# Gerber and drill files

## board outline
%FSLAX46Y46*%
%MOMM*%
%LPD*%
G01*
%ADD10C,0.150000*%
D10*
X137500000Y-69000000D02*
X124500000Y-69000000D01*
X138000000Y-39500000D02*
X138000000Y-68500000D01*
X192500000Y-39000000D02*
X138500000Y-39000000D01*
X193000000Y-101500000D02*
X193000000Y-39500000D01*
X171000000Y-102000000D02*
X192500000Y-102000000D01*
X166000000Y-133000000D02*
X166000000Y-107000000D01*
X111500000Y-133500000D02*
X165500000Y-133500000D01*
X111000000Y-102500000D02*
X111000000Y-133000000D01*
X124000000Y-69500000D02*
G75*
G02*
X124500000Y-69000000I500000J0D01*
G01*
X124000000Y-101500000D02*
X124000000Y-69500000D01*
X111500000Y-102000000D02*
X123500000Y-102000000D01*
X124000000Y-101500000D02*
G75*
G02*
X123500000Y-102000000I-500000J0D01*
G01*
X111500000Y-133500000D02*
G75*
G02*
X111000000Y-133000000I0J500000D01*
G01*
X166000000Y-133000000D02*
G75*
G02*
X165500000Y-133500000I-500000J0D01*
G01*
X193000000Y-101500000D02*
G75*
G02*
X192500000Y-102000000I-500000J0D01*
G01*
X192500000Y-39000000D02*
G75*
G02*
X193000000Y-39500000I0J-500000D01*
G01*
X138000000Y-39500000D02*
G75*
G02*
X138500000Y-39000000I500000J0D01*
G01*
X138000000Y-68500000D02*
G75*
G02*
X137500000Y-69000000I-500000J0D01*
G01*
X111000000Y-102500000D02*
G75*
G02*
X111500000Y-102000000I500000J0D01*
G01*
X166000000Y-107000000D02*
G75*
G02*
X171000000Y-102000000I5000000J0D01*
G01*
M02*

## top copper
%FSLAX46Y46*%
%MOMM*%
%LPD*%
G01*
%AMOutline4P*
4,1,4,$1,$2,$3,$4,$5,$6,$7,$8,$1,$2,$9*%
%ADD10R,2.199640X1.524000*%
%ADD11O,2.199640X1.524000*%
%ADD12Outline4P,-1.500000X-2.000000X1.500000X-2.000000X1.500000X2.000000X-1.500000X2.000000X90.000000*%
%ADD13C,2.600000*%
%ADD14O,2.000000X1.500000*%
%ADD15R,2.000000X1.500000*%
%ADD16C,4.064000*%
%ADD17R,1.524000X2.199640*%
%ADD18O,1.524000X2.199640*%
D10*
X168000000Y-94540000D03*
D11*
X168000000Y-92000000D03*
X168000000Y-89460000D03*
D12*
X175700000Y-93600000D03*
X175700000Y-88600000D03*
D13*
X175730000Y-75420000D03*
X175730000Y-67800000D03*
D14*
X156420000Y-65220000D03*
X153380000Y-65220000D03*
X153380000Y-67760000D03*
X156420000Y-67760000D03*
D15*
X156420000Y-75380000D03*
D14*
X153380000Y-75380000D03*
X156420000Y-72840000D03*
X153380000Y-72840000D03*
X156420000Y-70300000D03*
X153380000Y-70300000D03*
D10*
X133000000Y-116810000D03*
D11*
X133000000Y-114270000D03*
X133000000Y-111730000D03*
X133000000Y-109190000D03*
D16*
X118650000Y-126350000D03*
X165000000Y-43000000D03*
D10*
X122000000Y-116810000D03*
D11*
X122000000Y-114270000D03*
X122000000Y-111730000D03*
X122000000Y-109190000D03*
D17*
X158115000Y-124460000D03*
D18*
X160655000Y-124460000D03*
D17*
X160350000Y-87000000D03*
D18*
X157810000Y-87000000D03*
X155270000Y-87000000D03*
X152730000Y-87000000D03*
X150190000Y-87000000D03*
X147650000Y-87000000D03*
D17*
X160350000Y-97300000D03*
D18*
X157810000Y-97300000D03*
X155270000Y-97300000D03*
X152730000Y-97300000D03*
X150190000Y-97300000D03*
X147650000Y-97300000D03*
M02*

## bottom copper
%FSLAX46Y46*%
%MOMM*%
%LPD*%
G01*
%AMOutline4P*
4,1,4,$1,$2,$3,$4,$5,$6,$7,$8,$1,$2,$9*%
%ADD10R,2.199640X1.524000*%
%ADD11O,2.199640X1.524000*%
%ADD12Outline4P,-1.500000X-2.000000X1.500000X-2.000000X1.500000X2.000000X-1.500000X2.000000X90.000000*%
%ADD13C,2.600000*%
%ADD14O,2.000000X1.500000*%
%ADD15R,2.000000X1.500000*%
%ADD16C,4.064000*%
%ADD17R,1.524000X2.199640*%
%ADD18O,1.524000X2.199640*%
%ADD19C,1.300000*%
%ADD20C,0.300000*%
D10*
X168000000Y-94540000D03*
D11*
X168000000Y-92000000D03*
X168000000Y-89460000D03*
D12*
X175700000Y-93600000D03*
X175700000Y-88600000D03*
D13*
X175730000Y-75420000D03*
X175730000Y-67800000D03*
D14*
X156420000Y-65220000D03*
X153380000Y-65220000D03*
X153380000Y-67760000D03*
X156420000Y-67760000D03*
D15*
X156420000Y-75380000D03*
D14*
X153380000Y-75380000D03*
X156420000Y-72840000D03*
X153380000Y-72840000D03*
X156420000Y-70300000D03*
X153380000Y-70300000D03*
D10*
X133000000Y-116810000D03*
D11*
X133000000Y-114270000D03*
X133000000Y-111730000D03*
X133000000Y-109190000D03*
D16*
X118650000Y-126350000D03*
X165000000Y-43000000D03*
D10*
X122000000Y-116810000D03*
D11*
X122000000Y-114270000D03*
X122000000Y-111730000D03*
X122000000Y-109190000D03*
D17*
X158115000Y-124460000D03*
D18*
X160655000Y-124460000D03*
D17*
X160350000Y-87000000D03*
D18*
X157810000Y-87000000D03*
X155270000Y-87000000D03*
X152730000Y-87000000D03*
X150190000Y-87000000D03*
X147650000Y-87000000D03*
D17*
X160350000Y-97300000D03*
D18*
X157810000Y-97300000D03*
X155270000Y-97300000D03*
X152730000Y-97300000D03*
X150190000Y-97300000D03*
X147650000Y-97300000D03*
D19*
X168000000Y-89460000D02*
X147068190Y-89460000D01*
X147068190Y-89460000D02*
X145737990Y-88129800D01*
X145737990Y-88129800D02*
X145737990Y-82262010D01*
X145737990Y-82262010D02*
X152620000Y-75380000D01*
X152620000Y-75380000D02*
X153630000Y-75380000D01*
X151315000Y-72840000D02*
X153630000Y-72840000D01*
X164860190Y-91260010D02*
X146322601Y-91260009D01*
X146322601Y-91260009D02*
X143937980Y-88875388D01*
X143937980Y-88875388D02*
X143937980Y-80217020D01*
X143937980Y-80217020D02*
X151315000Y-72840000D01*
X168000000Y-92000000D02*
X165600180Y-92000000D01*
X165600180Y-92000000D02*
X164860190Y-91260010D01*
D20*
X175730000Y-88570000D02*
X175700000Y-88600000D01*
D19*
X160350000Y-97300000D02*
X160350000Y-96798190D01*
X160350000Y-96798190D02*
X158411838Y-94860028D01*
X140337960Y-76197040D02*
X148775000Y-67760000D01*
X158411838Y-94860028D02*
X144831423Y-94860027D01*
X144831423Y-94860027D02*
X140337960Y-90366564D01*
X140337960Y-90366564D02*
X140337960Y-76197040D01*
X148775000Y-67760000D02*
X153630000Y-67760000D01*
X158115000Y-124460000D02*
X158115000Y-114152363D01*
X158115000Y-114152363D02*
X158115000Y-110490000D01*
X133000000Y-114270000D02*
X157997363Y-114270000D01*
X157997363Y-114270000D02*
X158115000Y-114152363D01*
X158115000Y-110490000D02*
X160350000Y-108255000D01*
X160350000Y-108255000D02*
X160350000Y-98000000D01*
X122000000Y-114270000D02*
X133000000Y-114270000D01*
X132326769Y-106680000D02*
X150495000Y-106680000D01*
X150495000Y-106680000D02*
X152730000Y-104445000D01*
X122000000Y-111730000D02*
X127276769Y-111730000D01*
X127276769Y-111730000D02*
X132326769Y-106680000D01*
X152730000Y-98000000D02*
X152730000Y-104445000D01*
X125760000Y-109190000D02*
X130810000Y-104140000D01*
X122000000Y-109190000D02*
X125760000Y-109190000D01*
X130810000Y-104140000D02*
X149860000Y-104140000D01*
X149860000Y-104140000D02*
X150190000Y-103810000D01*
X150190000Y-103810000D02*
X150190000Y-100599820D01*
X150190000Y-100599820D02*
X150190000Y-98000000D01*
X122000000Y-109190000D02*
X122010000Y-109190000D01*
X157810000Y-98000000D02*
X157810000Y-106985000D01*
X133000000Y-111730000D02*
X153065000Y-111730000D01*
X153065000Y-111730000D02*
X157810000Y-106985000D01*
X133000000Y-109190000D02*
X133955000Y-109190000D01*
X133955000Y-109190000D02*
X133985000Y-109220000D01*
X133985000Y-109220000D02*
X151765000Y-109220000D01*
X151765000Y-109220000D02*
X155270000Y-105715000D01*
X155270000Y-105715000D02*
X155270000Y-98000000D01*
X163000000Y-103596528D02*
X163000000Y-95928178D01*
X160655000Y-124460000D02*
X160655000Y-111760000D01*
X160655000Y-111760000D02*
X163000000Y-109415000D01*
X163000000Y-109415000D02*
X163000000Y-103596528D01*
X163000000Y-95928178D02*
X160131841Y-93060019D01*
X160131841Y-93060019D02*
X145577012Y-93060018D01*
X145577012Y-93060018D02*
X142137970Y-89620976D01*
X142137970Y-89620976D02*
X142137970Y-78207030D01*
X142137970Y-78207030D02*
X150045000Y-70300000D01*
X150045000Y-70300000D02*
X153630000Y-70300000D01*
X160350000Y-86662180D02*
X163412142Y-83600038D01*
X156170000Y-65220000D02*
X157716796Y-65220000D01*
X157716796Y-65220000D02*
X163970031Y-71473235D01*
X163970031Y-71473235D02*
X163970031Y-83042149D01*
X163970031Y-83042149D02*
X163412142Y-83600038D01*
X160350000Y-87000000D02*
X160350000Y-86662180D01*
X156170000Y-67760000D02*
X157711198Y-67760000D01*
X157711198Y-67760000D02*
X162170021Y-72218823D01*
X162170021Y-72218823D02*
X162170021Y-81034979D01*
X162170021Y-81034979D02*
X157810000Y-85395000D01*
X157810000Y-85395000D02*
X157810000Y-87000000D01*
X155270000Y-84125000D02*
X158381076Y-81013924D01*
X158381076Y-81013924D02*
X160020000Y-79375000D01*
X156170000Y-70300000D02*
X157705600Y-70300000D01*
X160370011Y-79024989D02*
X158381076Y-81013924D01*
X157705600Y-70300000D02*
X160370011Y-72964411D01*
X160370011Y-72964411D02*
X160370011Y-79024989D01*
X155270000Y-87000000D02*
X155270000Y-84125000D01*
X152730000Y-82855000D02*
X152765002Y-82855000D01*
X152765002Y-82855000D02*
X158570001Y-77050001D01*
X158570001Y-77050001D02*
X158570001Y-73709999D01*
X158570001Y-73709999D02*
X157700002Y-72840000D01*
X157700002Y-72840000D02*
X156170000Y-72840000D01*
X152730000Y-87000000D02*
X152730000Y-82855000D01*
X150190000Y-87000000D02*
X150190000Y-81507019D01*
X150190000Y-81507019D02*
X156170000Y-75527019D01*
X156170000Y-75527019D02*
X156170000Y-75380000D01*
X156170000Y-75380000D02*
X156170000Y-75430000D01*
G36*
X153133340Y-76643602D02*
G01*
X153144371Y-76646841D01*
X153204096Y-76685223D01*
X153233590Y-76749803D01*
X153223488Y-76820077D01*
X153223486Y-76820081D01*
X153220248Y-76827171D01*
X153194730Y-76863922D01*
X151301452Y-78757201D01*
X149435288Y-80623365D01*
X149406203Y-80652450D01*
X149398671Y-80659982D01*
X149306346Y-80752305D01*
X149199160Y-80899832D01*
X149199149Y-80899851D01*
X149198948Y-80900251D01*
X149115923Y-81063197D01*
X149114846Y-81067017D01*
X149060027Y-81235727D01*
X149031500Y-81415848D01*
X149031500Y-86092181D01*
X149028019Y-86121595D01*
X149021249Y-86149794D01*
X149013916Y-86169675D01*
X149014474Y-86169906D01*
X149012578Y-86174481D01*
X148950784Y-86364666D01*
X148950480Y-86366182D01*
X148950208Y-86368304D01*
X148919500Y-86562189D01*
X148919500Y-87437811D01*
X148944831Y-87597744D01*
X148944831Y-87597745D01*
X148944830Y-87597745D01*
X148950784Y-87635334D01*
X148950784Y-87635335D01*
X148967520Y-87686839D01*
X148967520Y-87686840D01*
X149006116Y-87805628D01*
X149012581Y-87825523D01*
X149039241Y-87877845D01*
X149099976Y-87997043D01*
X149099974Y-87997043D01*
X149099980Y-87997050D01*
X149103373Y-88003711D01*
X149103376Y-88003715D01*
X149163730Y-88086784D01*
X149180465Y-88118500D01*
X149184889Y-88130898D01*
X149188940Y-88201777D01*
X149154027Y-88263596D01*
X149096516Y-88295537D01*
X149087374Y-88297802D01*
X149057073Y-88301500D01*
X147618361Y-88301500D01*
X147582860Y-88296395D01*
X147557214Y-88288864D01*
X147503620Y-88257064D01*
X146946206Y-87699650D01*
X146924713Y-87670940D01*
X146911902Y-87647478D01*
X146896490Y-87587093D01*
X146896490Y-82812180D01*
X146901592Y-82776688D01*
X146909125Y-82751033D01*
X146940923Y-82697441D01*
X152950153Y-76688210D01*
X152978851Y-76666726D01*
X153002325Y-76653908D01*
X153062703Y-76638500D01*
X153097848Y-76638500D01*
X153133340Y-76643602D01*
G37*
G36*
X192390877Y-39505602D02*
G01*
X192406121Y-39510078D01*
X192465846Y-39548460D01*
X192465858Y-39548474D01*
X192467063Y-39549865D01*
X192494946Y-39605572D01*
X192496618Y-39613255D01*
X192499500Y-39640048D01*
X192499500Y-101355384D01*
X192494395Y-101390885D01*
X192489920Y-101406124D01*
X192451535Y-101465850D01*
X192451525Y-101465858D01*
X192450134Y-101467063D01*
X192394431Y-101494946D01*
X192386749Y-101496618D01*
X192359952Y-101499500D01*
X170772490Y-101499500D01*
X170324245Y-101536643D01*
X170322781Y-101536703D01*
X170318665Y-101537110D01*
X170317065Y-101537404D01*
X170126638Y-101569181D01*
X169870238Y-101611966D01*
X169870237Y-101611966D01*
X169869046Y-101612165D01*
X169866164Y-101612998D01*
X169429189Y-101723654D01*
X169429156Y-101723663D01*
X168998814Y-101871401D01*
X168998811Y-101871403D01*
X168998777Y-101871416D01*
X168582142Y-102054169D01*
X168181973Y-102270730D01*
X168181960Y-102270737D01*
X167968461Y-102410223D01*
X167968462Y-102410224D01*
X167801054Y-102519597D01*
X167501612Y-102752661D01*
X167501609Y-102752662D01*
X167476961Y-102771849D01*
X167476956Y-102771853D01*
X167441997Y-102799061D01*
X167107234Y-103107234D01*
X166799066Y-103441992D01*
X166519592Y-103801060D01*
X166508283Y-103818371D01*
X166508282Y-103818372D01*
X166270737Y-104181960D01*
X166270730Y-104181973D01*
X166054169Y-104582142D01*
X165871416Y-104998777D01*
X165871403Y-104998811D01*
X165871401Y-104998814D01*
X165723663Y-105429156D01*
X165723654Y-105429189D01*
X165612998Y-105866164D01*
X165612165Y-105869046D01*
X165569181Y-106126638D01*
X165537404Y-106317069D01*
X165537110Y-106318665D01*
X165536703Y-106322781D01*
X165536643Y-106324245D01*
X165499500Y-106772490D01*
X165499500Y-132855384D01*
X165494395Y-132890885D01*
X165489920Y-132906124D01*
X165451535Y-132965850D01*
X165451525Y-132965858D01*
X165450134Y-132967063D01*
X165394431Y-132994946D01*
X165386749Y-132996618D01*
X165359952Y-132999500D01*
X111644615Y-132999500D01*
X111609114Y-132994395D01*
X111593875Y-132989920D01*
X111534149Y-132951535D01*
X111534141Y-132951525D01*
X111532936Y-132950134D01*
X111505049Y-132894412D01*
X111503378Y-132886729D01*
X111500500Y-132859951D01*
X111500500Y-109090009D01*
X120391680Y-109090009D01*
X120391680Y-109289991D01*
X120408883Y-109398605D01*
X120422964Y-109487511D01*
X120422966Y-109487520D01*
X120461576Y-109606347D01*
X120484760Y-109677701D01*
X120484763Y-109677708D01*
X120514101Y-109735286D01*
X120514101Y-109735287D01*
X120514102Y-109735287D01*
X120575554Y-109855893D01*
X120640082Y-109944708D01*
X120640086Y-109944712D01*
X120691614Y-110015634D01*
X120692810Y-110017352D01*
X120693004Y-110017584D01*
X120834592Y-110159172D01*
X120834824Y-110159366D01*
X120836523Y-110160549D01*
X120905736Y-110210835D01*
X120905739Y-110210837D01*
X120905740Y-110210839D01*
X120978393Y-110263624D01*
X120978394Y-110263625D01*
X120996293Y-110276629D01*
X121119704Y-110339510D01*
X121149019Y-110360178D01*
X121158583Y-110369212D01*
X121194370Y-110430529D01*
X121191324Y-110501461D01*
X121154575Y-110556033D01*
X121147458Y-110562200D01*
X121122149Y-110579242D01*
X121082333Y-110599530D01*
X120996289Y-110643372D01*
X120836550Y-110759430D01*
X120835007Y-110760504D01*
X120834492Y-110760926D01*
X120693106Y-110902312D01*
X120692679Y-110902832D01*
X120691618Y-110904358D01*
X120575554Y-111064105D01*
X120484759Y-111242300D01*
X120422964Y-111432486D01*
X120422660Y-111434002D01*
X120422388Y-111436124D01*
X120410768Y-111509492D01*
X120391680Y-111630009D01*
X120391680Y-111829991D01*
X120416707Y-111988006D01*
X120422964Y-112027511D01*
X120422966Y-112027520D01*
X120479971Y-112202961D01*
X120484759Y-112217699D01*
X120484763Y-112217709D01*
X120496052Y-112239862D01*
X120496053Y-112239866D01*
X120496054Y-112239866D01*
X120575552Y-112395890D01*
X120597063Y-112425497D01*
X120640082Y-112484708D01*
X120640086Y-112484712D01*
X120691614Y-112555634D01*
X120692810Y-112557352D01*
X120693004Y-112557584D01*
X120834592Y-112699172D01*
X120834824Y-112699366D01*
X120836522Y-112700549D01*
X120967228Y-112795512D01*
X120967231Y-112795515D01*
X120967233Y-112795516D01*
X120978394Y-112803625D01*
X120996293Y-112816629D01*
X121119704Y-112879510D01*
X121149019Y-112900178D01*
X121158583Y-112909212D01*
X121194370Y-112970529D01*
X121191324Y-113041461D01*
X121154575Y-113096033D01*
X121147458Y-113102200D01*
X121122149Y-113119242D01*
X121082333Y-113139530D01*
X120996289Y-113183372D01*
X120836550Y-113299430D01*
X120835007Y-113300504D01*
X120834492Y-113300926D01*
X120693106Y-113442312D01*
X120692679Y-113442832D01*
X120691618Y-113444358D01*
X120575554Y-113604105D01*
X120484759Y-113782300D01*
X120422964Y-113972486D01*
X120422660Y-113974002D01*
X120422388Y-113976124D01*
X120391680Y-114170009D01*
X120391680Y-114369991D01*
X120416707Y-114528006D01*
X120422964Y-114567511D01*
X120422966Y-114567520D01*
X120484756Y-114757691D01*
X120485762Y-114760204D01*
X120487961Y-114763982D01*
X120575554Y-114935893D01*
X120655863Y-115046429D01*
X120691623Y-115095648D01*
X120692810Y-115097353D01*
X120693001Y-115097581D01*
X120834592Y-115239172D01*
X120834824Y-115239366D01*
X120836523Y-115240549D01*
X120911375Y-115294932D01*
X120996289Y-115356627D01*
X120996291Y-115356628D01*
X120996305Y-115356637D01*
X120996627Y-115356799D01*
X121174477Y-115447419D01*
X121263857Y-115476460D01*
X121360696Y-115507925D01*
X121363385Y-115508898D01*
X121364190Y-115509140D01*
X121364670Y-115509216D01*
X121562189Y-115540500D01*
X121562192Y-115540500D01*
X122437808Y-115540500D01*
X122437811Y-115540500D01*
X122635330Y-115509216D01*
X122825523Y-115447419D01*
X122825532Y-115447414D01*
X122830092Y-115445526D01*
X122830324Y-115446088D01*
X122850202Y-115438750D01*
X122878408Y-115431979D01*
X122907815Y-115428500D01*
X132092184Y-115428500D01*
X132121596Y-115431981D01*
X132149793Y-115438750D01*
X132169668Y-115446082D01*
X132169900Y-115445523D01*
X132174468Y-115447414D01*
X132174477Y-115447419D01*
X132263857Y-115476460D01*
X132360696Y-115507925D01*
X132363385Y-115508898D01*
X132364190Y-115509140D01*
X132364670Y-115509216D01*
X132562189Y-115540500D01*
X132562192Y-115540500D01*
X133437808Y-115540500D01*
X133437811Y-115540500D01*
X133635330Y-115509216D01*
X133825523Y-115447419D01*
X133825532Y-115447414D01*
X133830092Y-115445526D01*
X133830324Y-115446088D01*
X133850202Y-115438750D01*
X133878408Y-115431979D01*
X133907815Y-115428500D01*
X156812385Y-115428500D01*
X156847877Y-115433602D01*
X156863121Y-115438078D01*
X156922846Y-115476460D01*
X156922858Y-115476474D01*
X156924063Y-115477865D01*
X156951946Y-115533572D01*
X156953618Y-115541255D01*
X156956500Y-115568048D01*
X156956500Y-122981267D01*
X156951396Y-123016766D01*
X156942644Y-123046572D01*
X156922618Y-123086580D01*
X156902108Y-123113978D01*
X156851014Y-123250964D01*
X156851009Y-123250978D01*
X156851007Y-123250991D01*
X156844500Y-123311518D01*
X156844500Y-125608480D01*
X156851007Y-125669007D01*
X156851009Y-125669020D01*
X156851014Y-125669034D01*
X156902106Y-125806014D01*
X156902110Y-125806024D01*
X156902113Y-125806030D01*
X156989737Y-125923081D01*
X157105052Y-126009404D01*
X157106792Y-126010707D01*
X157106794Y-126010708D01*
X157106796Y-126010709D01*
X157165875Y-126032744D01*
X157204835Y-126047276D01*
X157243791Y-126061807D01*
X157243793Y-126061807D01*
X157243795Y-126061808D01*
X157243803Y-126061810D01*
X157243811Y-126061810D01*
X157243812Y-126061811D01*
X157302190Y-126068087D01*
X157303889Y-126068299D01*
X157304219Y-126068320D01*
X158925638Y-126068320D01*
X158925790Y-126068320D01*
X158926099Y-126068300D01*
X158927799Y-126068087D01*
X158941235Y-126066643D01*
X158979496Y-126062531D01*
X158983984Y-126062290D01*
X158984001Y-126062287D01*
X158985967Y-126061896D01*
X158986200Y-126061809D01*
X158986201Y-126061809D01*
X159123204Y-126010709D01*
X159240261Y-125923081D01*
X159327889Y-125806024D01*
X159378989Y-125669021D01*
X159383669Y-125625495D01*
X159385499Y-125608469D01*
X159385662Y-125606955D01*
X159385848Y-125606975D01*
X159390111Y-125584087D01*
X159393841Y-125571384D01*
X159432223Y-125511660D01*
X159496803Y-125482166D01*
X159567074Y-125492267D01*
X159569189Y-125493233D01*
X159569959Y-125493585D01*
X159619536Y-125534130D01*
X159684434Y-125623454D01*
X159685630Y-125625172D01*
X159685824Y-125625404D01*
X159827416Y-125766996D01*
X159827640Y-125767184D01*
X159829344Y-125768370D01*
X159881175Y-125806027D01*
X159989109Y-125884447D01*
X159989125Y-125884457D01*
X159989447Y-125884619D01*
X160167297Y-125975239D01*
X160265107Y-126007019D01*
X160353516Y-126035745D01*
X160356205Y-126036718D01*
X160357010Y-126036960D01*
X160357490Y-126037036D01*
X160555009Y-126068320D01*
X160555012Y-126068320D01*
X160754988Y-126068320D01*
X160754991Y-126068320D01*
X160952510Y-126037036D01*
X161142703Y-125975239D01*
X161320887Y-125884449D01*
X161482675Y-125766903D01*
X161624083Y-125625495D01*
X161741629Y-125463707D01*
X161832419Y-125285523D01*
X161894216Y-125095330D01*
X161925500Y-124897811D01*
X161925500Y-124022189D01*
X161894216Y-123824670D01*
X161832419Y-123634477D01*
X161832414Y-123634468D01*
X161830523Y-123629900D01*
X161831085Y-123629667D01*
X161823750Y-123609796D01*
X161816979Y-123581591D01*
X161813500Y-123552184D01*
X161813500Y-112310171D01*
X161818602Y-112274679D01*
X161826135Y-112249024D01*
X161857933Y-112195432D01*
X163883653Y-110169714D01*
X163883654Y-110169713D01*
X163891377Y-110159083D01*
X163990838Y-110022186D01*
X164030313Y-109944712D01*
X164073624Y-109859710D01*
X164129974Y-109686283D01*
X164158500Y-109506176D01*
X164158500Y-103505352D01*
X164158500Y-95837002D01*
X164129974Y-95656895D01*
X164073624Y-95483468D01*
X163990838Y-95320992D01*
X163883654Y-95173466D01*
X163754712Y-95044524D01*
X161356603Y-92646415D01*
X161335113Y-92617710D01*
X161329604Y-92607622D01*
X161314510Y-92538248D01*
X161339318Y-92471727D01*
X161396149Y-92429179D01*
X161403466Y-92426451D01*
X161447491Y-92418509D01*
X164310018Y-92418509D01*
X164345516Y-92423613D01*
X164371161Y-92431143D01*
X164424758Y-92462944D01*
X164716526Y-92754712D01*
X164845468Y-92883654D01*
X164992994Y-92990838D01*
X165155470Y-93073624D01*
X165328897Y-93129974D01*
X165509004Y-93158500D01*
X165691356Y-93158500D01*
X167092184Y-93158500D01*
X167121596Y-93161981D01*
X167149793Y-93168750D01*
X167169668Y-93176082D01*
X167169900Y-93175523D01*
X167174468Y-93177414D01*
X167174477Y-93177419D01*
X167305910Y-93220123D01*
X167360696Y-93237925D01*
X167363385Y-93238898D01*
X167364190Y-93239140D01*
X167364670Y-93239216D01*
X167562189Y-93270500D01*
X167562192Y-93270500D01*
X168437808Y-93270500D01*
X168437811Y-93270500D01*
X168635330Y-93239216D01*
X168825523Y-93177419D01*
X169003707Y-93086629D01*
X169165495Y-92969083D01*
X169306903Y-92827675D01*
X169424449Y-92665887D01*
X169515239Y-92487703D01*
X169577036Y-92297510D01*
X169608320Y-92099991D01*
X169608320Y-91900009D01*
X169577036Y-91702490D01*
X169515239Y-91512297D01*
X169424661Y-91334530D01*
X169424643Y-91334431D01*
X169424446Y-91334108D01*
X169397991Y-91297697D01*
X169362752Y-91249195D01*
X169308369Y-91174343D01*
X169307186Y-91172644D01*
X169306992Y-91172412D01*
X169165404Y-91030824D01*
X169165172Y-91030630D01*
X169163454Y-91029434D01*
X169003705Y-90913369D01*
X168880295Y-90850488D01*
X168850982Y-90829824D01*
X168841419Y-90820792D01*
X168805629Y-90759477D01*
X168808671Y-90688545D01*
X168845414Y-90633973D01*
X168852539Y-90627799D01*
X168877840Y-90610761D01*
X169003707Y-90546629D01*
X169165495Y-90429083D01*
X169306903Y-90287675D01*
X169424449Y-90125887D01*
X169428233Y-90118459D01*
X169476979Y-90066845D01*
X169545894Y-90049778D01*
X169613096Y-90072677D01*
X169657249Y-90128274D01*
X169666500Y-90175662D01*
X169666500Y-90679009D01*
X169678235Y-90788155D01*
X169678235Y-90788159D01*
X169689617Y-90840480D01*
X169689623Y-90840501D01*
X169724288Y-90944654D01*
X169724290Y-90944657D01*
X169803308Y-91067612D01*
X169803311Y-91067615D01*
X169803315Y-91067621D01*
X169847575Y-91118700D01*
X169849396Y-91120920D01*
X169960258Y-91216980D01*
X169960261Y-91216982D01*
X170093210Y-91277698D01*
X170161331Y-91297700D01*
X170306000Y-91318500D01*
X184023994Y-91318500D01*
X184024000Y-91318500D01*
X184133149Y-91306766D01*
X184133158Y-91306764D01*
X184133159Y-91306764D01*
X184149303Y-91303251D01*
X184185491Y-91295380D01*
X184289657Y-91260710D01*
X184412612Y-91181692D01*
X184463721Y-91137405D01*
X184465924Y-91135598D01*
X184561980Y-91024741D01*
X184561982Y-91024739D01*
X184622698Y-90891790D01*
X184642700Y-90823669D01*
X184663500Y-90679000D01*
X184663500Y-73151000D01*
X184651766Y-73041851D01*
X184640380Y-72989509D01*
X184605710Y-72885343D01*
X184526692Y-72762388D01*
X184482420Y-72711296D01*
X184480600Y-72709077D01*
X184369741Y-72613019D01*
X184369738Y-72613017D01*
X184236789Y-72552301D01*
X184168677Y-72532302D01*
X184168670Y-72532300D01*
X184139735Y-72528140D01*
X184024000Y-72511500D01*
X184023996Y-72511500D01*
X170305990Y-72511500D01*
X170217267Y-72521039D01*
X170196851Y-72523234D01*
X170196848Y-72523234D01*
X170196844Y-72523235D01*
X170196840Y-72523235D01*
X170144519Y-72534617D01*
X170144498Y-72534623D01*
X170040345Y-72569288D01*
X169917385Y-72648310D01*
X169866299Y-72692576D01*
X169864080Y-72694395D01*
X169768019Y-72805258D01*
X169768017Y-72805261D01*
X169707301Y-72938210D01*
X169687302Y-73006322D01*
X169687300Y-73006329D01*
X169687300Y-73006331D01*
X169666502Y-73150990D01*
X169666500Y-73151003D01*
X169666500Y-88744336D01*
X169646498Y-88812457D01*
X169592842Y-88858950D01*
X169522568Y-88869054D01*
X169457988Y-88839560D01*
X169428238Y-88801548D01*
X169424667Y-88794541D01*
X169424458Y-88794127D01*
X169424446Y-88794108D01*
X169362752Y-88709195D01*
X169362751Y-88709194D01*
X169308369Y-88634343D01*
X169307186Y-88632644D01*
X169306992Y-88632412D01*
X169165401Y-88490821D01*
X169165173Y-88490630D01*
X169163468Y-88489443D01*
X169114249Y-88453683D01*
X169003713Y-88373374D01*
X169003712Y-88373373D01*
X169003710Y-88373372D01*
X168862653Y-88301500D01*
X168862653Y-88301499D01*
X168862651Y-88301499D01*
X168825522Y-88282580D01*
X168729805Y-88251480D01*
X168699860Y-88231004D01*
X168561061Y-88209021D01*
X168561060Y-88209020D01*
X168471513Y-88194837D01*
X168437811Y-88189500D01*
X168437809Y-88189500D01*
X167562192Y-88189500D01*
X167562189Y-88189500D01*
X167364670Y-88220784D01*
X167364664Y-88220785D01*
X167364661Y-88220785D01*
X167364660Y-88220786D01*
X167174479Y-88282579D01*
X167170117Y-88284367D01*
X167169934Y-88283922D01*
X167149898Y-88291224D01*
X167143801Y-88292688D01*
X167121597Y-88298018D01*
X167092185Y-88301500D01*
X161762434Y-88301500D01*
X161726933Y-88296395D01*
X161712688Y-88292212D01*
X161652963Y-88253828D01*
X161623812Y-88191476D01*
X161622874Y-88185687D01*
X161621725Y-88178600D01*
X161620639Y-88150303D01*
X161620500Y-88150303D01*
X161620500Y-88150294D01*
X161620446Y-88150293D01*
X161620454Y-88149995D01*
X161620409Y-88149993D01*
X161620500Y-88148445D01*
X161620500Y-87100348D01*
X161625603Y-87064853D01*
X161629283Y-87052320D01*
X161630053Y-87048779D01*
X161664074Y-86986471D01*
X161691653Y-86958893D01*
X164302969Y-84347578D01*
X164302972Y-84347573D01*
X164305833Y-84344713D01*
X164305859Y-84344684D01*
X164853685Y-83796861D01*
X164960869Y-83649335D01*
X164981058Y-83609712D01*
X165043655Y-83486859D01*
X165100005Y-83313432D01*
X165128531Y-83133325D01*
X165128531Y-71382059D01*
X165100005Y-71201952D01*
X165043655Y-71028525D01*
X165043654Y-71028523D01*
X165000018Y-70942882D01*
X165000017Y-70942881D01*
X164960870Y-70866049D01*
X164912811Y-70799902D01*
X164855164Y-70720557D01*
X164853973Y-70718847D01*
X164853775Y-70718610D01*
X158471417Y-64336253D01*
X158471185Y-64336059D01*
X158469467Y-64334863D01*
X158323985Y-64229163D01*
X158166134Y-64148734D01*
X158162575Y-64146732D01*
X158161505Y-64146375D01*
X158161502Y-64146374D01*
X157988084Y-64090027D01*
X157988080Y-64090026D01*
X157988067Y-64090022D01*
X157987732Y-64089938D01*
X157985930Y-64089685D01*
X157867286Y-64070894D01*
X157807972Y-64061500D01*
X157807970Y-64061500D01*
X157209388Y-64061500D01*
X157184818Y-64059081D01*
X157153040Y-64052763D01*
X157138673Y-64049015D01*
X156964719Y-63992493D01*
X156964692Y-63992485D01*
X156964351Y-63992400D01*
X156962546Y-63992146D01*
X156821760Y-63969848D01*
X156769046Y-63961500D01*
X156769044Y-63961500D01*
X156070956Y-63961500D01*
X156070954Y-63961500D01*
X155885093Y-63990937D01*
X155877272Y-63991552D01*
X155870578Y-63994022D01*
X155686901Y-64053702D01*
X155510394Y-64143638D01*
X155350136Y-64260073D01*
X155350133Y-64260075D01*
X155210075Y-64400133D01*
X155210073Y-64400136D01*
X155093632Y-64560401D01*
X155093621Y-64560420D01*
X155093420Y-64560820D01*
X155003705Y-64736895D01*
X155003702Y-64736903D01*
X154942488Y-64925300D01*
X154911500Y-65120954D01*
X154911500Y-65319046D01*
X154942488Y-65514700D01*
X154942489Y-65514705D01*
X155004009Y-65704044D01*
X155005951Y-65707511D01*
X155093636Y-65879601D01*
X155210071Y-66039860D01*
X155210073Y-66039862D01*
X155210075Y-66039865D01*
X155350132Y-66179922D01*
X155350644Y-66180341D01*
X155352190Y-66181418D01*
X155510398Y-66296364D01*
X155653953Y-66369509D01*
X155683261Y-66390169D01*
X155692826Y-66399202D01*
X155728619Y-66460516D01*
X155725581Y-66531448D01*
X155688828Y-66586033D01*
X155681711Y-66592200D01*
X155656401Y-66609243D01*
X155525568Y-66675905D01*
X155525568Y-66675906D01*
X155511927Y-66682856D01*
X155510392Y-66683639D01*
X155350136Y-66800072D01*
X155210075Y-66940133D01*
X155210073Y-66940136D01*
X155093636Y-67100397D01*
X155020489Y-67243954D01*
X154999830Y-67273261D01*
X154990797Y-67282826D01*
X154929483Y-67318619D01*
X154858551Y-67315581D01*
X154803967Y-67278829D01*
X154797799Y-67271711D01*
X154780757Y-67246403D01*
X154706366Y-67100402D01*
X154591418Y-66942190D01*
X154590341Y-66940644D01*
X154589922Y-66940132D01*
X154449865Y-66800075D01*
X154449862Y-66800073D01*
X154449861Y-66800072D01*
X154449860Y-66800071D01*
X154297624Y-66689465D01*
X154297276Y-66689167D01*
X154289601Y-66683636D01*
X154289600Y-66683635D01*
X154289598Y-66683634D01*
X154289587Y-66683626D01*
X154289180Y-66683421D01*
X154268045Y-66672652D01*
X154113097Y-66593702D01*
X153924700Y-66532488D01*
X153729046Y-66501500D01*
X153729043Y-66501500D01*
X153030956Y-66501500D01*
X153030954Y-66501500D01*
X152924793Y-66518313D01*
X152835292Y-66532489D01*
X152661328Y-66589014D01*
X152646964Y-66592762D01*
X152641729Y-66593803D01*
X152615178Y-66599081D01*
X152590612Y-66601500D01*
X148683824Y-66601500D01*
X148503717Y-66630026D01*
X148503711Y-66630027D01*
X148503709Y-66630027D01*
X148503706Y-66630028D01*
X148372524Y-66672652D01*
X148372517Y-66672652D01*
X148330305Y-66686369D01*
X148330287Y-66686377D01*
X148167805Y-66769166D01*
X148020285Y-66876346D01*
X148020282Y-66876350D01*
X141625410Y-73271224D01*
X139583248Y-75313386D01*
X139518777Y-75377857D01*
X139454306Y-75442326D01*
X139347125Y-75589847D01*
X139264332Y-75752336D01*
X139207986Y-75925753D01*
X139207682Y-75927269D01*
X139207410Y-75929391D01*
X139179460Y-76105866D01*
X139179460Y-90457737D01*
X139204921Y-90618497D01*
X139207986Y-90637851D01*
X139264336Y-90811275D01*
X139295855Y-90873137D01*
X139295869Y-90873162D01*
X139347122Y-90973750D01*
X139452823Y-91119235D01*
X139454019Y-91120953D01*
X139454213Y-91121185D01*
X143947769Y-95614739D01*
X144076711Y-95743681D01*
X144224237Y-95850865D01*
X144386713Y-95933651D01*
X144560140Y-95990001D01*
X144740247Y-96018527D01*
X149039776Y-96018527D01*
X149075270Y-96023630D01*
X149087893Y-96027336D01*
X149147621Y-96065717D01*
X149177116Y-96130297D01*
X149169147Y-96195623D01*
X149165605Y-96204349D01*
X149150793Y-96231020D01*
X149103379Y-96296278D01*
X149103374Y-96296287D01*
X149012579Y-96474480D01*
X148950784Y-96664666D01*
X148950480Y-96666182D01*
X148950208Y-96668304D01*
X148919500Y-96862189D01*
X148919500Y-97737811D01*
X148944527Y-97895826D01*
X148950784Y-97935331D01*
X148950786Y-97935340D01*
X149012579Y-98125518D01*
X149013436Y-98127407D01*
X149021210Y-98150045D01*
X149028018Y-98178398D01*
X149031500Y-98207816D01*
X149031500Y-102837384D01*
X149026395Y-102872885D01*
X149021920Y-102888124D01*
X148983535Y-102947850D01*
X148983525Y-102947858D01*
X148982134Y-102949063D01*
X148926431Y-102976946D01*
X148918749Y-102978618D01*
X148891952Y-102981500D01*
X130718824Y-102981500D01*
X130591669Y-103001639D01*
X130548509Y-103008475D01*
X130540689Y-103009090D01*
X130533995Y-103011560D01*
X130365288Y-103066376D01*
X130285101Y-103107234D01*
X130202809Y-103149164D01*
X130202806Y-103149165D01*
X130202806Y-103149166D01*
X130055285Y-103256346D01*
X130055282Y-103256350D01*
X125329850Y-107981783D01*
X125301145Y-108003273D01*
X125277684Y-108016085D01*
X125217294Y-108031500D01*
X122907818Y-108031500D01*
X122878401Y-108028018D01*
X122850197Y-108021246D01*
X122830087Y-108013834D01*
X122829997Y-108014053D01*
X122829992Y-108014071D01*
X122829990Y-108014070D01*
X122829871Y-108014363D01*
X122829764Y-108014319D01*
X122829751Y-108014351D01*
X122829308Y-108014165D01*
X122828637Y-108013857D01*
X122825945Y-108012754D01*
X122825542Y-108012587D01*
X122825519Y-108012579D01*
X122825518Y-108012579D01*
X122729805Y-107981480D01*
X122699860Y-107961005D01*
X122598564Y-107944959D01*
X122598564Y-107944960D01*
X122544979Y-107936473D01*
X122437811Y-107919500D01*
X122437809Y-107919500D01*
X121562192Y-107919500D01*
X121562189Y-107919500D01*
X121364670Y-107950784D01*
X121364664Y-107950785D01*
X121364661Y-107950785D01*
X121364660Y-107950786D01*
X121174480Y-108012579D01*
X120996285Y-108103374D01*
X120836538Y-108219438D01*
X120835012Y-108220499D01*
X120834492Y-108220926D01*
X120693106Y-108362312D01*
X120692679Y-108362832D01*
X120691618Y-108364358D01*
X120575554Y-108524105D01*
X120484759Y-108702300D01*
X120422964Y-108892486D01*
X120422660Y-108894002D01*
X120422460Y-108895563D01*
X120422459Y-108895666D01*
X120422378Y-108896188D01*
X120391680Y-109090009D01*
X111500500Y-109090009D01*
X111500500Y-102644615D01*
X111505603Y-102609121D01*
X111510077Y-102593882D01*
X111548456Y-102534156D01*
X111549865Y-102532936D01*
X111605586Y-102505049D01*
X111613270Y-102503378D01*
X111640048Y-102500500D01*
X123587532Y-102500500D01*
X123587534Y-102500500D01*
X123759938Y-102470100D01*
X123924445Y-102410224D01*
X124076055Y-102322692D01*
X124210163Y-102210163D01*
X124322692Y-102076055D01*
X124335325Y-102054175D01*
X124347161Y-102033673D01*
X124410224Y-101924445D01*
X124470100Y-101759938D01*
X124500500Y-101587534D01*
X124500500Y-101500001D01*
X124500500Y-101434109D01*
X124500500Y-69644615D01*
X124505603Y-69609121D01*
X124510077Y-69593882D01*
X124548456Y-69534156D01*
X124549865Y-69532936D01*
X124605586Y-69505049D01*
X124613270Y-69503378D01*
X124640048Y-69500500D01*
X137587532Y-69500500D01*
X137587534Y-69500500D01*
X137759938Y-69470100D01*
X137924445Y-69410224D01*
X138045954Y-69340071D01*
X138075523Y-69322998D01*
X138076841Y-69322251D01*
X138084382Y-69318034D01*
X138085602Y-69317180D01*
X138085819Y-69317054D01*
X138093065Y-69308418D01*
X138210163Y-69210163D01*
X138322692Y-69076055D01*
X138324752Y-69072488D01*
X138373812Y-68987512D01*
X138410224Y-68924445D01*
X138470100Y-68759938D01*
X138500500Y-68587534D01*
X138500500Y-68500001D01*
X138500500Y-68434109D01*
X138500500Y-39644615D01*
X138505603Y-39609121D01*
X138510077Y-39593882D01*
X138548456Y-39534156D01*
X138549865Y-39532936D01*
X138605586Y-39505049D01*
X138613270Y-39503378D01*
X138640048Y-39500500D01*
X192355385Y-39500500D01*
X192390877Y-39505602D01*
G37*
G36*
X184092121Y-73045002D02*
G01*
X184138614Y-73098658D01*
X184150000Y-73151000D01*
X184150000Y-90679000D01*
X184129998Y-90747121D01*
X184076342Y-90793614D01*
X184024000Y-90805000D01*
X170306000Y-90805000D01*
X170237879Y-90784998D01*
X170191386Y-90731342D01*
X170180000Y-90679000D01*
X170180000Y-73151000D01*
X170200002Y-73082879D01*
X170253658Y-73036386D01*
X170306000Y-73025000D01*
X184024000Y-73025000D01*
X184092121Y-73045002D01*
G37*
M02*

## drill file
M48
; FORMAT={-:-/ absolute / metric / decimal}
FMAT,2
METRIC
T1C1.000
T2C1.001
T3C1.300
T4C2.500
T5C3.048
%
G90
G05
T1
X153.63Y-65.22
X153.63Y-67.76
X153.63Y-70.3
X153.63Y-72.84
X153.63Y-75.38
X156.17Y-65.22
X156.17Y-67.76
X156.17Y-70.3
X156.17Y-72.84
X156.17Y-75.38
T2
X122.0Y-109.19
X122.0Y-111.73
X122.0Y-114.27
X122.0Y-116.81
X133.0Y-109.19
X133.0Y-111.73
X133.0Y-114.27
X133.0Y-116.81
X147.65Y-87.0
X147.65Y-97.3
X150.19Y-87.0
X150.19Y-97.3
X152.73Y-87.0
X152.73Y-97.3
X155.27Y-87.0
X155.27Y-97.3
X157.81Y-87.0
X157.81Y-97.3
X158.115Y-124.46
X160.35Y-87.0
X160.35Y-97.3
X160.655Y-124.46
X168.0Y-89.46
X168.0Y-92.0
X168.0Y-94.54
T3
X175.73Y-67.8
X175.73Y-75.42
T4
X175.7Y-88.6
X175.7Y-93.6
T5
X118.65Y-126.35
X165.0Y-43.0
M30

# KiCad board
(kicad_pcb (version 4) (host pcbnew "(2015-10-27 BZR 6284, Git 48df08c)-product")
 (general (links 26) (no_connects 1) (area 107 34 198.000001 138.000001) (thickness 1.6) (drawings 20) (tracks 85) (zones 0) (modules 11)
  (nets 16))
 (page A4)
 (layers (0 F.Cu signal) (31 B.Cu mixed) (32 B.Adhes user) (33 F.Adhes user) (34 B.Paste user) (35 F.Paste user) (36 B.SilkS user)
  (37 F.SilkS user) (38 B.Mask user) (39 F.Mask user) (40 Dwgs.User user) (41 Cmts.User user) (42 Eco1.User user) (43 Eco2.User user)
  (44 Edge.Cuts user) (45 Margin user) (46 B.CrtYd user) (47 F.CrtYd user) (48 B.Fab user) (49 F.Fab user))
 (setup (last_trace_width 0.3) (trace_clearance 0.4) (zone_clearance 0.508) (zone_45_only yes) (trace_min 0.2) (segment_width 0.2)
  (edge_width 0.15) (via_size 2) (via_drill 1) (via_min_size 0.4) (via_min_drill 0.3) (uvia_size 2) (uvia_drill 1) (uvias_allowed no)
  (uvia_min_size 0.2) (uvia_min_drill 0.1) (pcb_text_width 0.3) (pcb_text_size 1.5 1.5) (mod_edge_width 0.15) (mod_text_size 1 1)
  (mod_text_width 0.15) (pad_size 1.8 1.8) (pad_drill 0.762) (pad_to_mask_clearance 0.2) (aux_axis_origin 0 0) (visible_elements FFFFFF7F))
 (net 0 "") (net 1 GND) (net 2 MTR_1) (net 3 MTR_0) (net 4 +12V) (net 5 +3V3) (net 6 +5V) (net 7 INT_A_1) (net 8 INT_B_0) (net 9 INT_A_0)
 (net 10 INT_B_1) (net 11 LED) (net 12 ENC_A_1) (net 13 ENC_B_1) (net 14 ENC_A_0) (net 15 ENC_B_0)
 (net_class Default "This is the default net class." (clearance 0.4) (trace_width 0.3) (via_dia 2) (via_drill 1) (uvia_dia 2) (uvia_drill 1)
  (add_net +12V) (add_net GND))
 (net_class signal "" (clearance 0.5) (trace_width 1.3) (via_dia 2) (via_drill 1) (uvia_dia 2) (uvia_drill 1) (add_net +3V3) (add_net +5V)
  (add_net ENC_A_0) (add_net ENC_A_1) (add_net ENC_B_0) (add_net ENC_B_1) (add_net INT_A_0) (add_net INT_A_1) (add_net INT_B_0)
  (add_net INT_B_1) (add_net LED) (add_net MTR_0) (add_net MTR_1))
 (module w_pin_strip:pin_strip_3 (layer F.Cu) (at 168 92 90)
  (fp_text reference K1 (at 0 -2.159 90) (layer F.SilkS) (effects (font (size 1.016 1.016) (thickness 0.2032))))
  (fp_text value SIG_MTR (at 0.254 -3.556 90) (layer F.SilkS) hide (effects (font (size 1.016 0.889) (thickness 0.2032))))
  (pad 1 thru_hole rect (at -2.54 0 90) (size 1.524 2.19964) (drill 1.00076) (layers *.Cu *.Mask F.SilkS) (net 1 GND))
  (pad 2 thru_hole oval (at 0 0 90) (size 1.524 2.19964) (drill 1.00076) (layers *.Cu *.Mask F.SilkS) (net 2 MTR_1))
  (pad 3 thru_hole oval (at 2.54 0 90) (size 1.524 2.19964) (drill 1.00076) (layers *.Cu *.Mask F.SilkS) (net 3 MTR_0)))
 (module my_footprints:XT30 (layer F.Cu) (at 175.7 91.1 90)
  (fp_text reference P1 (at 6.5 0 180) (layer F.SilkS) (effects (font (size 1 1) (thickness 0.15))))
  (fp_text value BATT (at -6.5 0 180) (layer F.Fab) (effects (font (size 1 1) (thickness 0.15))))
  (pad 1 thru_hole trapezoid (at -2.5 0 90) (size 3 4) (drill 2.5) (layers *.Cu *.Mask F.SilkS) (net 1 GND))
  (pad 2 thru_hole trapezoid (at 2.5 0 90) (size 3 4) (drill 2.5) (layers *.Cu *.Mask F.SilkS) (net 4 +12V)))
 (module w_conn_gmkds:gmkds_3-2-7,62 (layer F.Cu) (at 175.73 71.61 90)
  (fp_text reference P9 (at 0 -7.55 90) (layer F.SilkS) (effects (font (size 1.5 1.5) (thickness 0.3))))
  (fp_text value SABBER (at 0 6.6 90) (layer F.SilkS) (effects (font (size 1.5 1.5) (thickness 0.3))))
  (pad 1 thru_hole circle (at -3.81 0 90) (size 2.6 2.6) (drill 1.3) (layers *.Cu *.Mask F.SilkS) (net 4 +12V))
  (pad 2 thru_hole circle (at 3.81 0 90) (size 2.6 2.6) (drill 1.3) (layers *.Cu *.Mask F.SilkS) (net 1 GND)))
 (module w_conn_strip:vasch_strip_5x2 (layer F.Cu) (at 154.9 70.3 90)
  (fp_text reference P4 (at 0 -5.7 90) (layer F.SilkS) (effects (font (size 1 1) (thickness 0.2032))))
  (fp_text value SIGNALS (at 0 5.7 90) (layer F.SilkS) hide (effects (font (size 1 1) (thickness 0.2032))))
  (pad 9 thru_hole oval (at 5.08 1.27 90) (size 1.5 2) (drill 1 (offset 0 0.25)) (layers *.Cu *.Mask F.SilkS) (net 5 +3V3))
  (pad 10 thru_hole oval (at 5.08 -1.27 90) (size 1.5 2) (drill 1 (offset 0 -0.25)) (layers *.Cu *.Mask F.SilkS) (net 1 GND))
  (pad 8 thru_hole oval (at 2.54 -1.27 90) (size 1.5 2) (drill 1 (offset 0 -0.25)) (layers *.Cu *.Mask F.SilkS) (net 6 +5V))
  (pad 7 thru_hole oval (at 2.54 1.27 90) (size 1.5 2) (drill 1 (offset 0 0.25)) (layers *.Cu *.Mask F.SilkS) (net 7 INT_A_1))
  (pad 1 thru_hole rect (at -5.08 1.27 90) (size 1.5 2) (drill 1 (offset 0 0.25)) (layers *.Cu *.Mask F.SilkS) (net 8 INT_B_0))
  (pad 2 thru_hole oval (at -5.08 -1.27 90) (size 1.5 2) (drill 1 (offset 0 -0.25)) (layers *.Cu *.Mask F.SilkS) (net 3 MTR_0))
  (pad 3 thru_hole oval (at -2.54 1.27 90) (size 1.5 2) (drill 1 (offset 0 0.25)) (layers *.Cu *.Mask F.SilkS) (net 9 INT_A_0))
  (pad 4 thru_hole oval (at -2.54 -1.27 90) (size 1.5 2) (drill 1 (offset 0 -0.25)) (layers *.Cu *.Mask F.SilkS) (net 2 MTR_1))
  (pad 5 thru_hole oval (at 0 1.27 90) (size 1.5 2) (drill 1 (offset 0 0.25)) (layers *.Cu *.Mask F.SilkS) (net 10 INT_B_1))
  (pad 6 thru_hole oval (at 0 -1.27 90) (size 1.5 2) (drill 1 (offset 0 -0.25)) (layers *.Cu *.Mask F.SilkS) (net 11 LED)))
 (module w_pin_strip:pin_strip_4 (layer F.Cu) (at 133 113 90)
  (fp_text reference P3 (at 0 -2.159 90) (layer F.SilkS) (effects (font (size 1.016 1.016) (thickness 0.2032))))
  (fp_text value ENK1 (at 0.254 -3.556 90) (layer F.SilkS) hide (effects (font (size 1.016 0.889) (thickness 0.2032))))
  (pad 1 thru_hole rect (at -3.81 0 90) (size 1.524 2.19964) (drill 1.00076) (layers *.Cu *.Mask F.SilkS) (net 1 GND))
  (pad 2 thru_hole oval (at -1.27 0 90) (size 1.524 2.19964) (drill 1.00076) (layers *.Cu *.Mask F.SilkS) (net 6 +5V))
  (pad 3 thru_hole oval (at 1.27 0 90) (size 1.524 2.19964) (drill 1.00076) (layers *.Cu *.Mask F.SilkS) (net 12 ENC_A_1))
  (pad 4 thru_hole oval (at 3.81 0 90) (size 1.524 2.19964) (drill 1.00076) (layers *.Cu *.Mask F.SilkS) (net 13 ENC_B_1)))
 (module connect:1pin (layer F.Cu) (at 118.65 126.35)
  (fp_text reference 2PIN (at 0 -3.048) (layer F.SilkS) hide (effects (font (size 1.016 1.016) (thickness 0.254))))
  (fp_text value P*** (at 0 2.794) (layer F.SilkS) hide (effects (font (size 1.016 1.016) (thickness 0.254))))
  (pad 1 thru_hole circle (at 0 0) (size 4.064 4.064) (drill 3.048) (layers *.Cu *.Mask F.SilkS) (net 1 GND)))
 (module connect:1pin (layer F.Cu) (at 165 43)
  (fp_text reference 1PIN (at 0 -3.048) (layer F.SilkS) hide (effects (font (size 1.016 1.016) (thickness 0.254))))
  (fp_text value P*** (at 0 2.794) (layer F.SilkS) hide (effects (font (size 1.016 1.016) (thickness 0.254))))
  (pad 2 thru_hole circle (at 0 0) (size 4.064 4.064) (drill 3.048) (layers *.Cu *.Mask F.SilkS) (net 1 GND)))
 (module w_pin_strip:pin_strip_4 (layer F.Cu) (at 122 113 90)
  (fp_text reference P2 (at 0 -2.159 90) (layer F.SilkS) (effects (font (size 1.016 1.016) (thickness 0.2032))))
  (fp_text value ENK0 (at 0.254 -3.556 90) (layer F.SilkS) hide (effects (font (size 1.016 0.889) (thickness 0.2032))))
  (pad 1 thru_hole rect (at -3.81 0 90) (size 1.524 2.19964) (drill 1.00076) (layers *.Cu *.Mask F.SilkS) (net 1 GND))
  (pad 2 thru_hole oval (at -1.27 0 90) (size 1.524 2.19964) (drill 1.00076) (layers *.Cu *.Mask F.SilkS) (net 6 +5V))
  (pad 3 thru_hole oval (at 1.27 0 90) (size 1.524 2.19964) (drill 1.00076) (layers *.Cu *.Mask F.SilkS) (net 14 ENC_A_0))
  (pad 4 thru_hole oval (at 3.81 0 90) (size 1.524 2.19964) (drill 1.00076) (layers *.Cu *.Mask F.SilkS) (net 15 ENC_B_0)))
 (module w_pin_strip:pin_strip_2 (layer F.Cu) (at 159.385 124.46)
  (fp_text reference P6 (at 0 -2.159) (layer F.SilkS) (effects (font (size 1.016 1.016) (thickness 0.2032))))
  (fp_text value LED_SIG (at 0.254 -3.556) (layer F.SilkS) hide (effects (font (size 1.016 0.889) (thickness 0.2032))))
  (pad 1 thru_hole rect (at -1.27 0) (size 1.524 2.19964) (drill 1.00076) (layers *.Cu *.Mask F.SilkS) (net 6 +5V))
  (pad 2 thru_hole oval (at 1.27 0) (size 1.524 2.19964) (drill 1.00076) (layers *.Cu *.Mask F.SilkS) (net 11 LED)))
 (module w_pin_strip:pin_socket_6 (layer F.Cu) (at 154 87 180)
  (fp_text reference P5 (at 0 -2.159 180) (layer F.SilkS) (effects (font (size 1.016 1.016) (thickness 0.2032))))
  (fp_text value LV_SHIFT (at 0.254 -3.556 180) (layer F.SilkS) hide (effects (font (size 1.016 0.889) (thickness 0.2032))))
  (pad 1 thru_hole rect (at -6.35 0 180) (size 1.524 2.19964) (drill 1.00076) (layers *.Cu *.Mask F.SilkS) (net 5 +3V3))
  (pad 2 thru_hole oval (at -3.81 0 180) (size 1.524 2.19964) (drill 1.00076) (layers *.Cu *.Mask F.SilkS) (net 7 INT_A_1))
  (pad 3 thru_hole oval (at -1.27 0 180) (size 1.524 2.19964) (drill 1.00076) (layers *.Cu *.Mask F.SilkS) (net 10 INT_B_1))
  (pad 4 thru_hole oval (at 1.27 0 180) (size 1.524 2.19964) (drill 1.00076) (layers *.Cu *.Mask F.SilkS) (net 9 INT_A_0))
  (pad 5 thru_hole oval (at 3.81 0 180) (size 1.524 2.19964) (drill 1.00076) (layers *.Cu *.Mask F.SilkS) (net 8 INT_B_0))
  (pad 6 thru_hole oval (at 6.35 0 180) (size 1.524 2.19964) (drill 1.00076) (layers *.Cu *.Mask F.SilkS) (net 1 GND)))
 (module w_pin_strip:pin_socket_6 (layer F.Cu) (at 154 97.3 180)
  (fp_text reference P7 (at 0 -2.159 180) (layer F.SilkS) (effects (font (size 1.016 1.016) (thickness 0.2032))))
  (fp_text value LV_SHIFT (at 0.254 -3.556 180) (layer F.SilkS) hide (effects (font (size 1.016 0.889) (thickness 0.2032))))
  (pad 1 thru_hole rect (at -6.35 0 180) (size 1.524 2.19964) (drill 1.00076) (layers *.Cu *.Mask F.SilkS) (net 6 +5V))
  (pad 2 thru_hole oval (at -3.81 0 180) (size 1.524 2.19964) (drill 1.00076) (layers *.Cu *.Mask F.SilkS) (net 12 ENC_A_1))
  (pad 3 thru_hole oval (at -1.27 0 180) (size 1.524 2.19964) (drill 1.00076) (layers *.Cu *.Mask F.SilkS) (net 13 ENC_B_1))
  (pad 4 thru_hole oval (at 1.27 0 180) (size 1.524 2.19964) (drill 1.00076) (layers *.Cu *.Mask F.SilkS) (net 14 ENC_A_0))
  (pad 5 thru_hole oval (at 3.81 0 180) (size 1.524 2.19964) (drill 1.00076) (layers *.Cu *.Mask F.SilkS) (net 15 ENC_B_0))
  (pad 6 thru_hole oval (at 6.35 0 180) (size 1.524 2.19964) (drill 1.00076) (layers *.Cu *.Mask F.SilkS) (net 1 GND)))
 (gr_line (start 137.5 69) (end 124.5 69) (angle 90) (layer Edge.Cuts) (width 0.15))
 (gr_line (start 138 39.5) (end 138 68.5) (angle 90) (layer Edge.Cuts) (width 0.15))
 (gr_line (start 192.5 39) (end 138.5 39) (angle 90) (layer Edge.Cuts) (width 0.15))
 (gr_line (start 193 101.5) (end 193 39.5) (angle 90) (layer Edge.Cuts) (width 0.15))
 (gr_line (start 171 102) (end 192.5 102) (angle 90) (layer Edge.Cuts) (width 0.15))
 (gr_line (start 166 133) (end 166 107) (angle 90) (layer Edge.Cuts) (width 0.15))
 (gr_line (start 111.5 133.5) (end 165.5 133.5) (angle 90) (layer Edge.Cuts) (width 0.15))
 (gr_line (start 111 102.5) (end 111 133) (angle 90) (layer Edge.Cuts) (width 0.15))
 (gr_arc (start 124.5 69.5) (end 124 69.5) (angle 90) (layer Edge.Cuts) (width 0.15))
 (gr_line (start 124 101.5) (end 124 69.5) (angle 90) (layer Edge.Cuts) (width 0.15))
 (gr_line (start 111.5 102) (end 123.5 102) (angle 90) (layer Edge.Cuts) (width 0.15))
 (gr_arc (start 123.5 101.5) (end 124 101.5) (angle 90) (layer Edge.Cuts) (width 0.15))
 (gr_arc (start 111.5 133) (end 111.5 133.5) (angle 90) (layer Edge.Cuts) (width 0.15))
 (gr_arc (start 165.5 133) (end 166 133) (angle 90) (layer Edge.Cuts) (width 0.15))
 (gr_arc (start 192.5 101.5) (end 193 101.5) (angle 90) (layer Edge.Cuts) (width 0.15))
 (gr_arc (start 192.5 39.5) (end 192.5 39) (angle 90) (layer Edge.Cuts) (width 0.15))
 (gr_arc (start 138.5 39.5) (end 138 39.5) (angle 90) (layer Edge.Cuts) (width 0.15))
 (gr_arc (start 137.5 68.5) (end 138 68.5) (angle 90) (layer Edge.Cuts) (width 0.15))
 (gr_arc (start 111.5 102.5) (end 111 102.5) (angle 90) (layer Edge.Cuts) (width 0.15))
 (gr_arc (start 171 107) (end 166 107) (angle 90) (layer Edge.Cuts) (width 0.15))
 (segment (start 168 89.46) (end 147.06819 89.46) (width 1.3) (layer B.Cu) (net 3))
 (segment (start 147.06819 89.46) (end 145.73799 88.1298) (width 1.3) (layer B.Cu) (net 3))
 (segment (start 145.73799 88.1298) (end 145.73799 82.26201) (width 1.3) (layer B.Cu) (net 3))
 (segment (start 145.73799 82.26201) (end 152.62 75.38) (width 1.3) (layer B.Cu) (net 3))
 (segment (start 152.62 75.38) (end 153.63 75.38) (width 1.3) (layer B.Cu) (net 3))
 (segment (start 151.315 72.84) (end 153.63 72.84) (width 1.3) (layer B.Cu) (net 2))
 (segment (start 164.86019 91.26001) (end 146.322601 91.260009) (width 1.3) (layer B.Cu) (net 2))
 (segment (start 146.322601 91.260009) (end 143.93798 88.875388) (width 1.3) (layer B.Cu) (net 2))
 (segment (start 143.93798 88.875388) (end 143.93798 80.21702) (width 1.3) (layer B.Cu) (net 2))
 (segment (start 143.93798 80.21702) (end 151.315 72.84) (width 1.3) (layer B.Cu) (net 2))
 (segment (start 168 92) (end 165.60018 92) (width 1.3) (layer B.Cu) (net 2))
 (segment (start 165.60018 92) (end 164.86019 91.26001) (width 1.3) (layer B.Cu) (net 2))
 (segment (start 175.73 88.57) (end 175.7 88.6) (width 0.3) (layer B.Cu) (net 4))
 (segment (start 160.35 97.3) (end 160.35 96.79819) (width 1.3) (layer B.Cu) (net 6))
 (segment (start 160.35 96.79819) (end 158.411838 94.860028) (width 1.3) (layer B.Cu) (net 6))
 (segment (start 140.33796 76.19704) (end 148.775 67.76) (width 1.3) (layer B.Cu) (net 6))
 (segment (start 158.411838 94.860028) (end 144.831423 94.860027) (width 1.3) (layer B.Cu) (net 6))
 (segment (start 144.831423 94.860027) (end 140.33796 90.366564) (width 1.3) (layer B.Cu) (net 6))
 (segment (start 140.33796 90.366564) (end 140.33796 76.19704) (width 1.3) (layer B.Cu) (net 6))
 (segment (start 148.775 67.76) (end 153.63 67.76) (width 1.3) (layer B.Cu) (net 6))
 (segment (start 158.115 124.46) (end 158.115 114.152363) (width 1.3) (layer B.Cu) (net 6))
 (segment (start 158.115 114.152363) (end 158.115 110.49) (width 1.3) (layer B.Cu) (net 6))
 (segment (start 133 114.27) (end 157.997363 114.27) (width 1.3) (layer B.Cu) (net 6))
 (segment (start 157.997363 114.27) (end 158.115 114.152363) (width 1.3) (layer B.Cu) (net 6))
 (segment (start 158.115 110.49) (end 160.35 108.255) (width 1.3) (layer B.Cu) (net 6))
 (segment (start 160.35 108.255) (end 160.35 98) (width 1.3) (layer B.Cu) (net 6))
 (segment (start 122 114.27) (end 133 114.27) (width 1.3) (layer B.Cu) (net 6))
 (segment (start 132.326769 106.68) (end 150.495 106.68) (width 1.3) (layer B.Cu) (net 14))
 (segment (start 150.495 106.68) (end 152.73 104.445) (width 1.3) (layer B.Cu) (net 14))
 (segment (start 122 111.73) (end 127.276769 111.73) (width 1.3) (layer B.Cu) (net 14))
 (segment (start 127.276769 111.73) (end 132.326769 106.68) (width 1.3) (layer B.Cu) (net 14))
 (segment (start 152.73 98) (end 152.73 104.445) (width 1.3) (layer B.Cu) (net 14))
 (segment (start 125.76 109.19) (end 130.81 104.14) (width 1.3) (layer B.Cu) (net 15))
 (segment (start 122 109.19) (end 125.76 109.19) (width 1.3) (layer B.Cu) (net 15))
 (segment (start 130.81 104.14) (end 149.86 104.14) (width 1.3) (layer B.Cu) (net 15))
 (segment (start 149.86 104.14) (end 150.19 103.81) (width 1.3) (layer B.Cu) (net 15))
 (segment (start 150.19 103.81) (end 150.19 100.59982) (width 1.3) (layer B.Cu) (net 15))
 (segment (start 150.19 100.59982) (end 150.19 98) (width 1.3) (layer B.Cu) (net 15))
 (segment (start 122 109.19) (end 122.01 109.19) (width 1.3) (layer B.Cu) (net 15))
 (segment (start 157.81 98) (end 157.81 106.985) (width 1.3) (layer B.Cu) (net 12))
 (segment (start 133 111.73) (end 153.065 111.73) (width 1.3) (layer B.Cu) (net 12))
 (segment (start 153.065 111.73) (end 157.81 106.985) (width 1.3) (layer B.Cu) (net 12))
 (segment (start 133 109.19) (end 133.955 109.19) (width 1.3) (layer B.Cu) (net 13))
 (segment (start 133.955 109.19) (end 133.985 109.22) (width 1.3) (layer B.Cu) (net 13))
 (segment (start 133.985 109.22) (end 151.765 109.22) (width 1.3) (layer B.Cu) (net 13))
 (segment (start 151.765 109.22) (end 155.27 105.715) (width 1.3) (layer B.Cu) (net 13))
 (segment (start 155.27 105.715) (end 155.27 98) (width 1.3) (layer B.Cu) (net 13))
 (segment (start 163 103.596528) (end 163 95.928178) (width 1.3) (layer B.Cu) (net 11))
 (segment (start 160.655 124.46) (end 160.655 111.76) (width 1.3) (layer B.Cu) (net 11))
 (segment (start 160.655 111.76) (end 163 109.415) (width 1.3) (layer B.Cu) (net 11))
 (segment (start 163 109.415) (end 163 103.596528) (width 1.3) (layer B.Cu) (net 11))
 (segment (start 163 95.928178) (end 160.131841 93.060019) (width 1.3) (layer B.Cu) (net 11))
 (segment (start 160.131841 93.060019) (end 145.577012 93.060018) (width 1.3) (layer B.Cu) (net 11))
 (segment (start 145.577012 93.060018) (end 142.13797 89.620976) (width 1.3) (layer B.Cu) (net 11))
 (segment (start 142.13797 89.620976) (end 142.13797 78.20703) (width 1.3) (layer B.Cu) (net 11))
 (segment (start 142.13797 78.20703) (end 150.045 70.3) (width 1.3) (layer B.Cu) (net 11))
 (segment (start 150.045 70.3) (end 153.63 70.3) (width 1.3) (layer B.Cu) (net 11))
 (segment (start 160.35 86.66218) (end 163.412142 83.600038) (width 1.3) (layer B.Cu) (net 5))
 (segment (start 156.17 65.22) (end 157.716796 65.22) (width 1.3) (layer B.Cu) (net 5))
 (segment (start 157.716796 65.22) (end 163.970031 71.473235) (width 1.3) (layer B.Cu) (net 5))
 (segment (start 163.970031 71.473235) (end 163.970031 83.042149) (width 1.3) (layer B.Cu) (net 5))
 (segment (start 163.970031 83.042149) (end 163.412142 83.600038) (width 1.3) (layer B.Cu) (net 5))
 (segment (start 160.35 87) (end 160.35 86.66218) (width 1.3) (layer B.Cu) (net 5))
 (segment (start 156.17 67.76) (end 157.711198 67.76) (width 1.3) (layer B.Cu) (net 7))
 (segment (start 157.711198 67.76) (end 162.170021 72.218823) (width 1.3) (layer B.Cu) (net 7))
 (segment (start 162.170021 72.218823) (end 162.170021 81.034979) (width 1.3) (layer B.Cu) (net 7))
 (segment (start 162.170021 81.034979) (end 157.81 85.395) (width 1.3) (layer B.Cu) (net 7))
 (segment (start 157.81 85.395) (end 157.81 87) (width 1.3) (layer B.Cu) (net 7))
 (segment (start 155.27 84.125) (end 158.381076 81.013924) (width 1.3) (layer B.Cu) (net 10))
 (segment (start 158.381076 81.013924) (end 160.02 79.375) (width 1.3) (layer B.Cu) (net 10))
 (segment (start 156.17 70.3) (end 157.7056 70.3) (width 1.3) (layer B.Cu) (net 10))
 (segment (start 160.370011 79.024989) (end 158.381076 81.013924) (width 1.3) (layer B.Cu) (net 10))
 (segment (start 157.7056 70.3) (end 160.370011 72.964411) (width 1.3) (layer B.Cu) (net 10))
 (segment (start 160.370011 72.964411) (end 160.370011 79.024989) (width 1.3) (layer B.Cu) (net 10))
 (segment (start 155.27 87) (end 155.27 84.125) (width 1.3) (layer B.Cu) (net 10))
 (segment (start 152.73 82.855) (end 152.765002 82.855) (width 1.3) (layer B.Cu) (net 9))
 (segment (start 152.765002 82.855) (end 158.570001 77.050001) (width 1.3) (layer B.Cu) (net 9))
 (segment (start 158.570001 77.050001) (end 158.570001 73.709999) (width 1.3) (layer B.Cu) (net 9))
 (segment (start 158.570001 73.709999) (end 157.700002 72.84) (width 1.3) (layer B.Cu) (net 9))
 (segment (start 157.700002 72.84) (end 156.17 72.84) (width 1.3) (layer B.Cu) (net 9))
 (segment (start 152.73 87) (end 152.73 82.855) (width 1.3) (layer B.Cu) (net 9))
 (segment (start 150.19 87) (end 150.19 81.507019) (width 1.3) (layer B.Cu) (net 8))
 (segment (start 150.19 81.507019) (end 156.17 75.527019) (width 1.3) (layer B.Cu) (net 8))
 (segment (start 156.17 75.527019) (end 156.17 75.38) (width 1.3) (layer B.Cu) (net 8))
 (segment (start 156.17 75.38) (end 156.17 75.43) (width 1.3) (layer B.Cu) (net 8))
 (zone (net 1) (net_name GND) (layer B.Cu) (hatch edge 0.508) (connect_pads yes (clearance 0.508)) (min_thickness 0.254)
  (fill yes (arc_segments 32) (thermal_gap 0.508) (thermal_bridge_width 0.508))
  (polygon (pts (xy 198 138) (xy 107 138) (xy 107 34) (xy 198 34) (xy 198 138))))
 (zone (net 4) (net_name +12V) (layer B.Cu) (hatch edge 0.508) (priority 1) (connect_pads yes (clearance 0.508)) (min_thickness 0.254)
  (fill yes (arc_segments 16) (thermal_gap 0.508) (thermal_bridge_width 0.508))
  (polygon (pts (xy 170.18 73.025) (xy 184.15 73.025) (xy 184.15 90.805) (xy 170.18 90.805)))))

